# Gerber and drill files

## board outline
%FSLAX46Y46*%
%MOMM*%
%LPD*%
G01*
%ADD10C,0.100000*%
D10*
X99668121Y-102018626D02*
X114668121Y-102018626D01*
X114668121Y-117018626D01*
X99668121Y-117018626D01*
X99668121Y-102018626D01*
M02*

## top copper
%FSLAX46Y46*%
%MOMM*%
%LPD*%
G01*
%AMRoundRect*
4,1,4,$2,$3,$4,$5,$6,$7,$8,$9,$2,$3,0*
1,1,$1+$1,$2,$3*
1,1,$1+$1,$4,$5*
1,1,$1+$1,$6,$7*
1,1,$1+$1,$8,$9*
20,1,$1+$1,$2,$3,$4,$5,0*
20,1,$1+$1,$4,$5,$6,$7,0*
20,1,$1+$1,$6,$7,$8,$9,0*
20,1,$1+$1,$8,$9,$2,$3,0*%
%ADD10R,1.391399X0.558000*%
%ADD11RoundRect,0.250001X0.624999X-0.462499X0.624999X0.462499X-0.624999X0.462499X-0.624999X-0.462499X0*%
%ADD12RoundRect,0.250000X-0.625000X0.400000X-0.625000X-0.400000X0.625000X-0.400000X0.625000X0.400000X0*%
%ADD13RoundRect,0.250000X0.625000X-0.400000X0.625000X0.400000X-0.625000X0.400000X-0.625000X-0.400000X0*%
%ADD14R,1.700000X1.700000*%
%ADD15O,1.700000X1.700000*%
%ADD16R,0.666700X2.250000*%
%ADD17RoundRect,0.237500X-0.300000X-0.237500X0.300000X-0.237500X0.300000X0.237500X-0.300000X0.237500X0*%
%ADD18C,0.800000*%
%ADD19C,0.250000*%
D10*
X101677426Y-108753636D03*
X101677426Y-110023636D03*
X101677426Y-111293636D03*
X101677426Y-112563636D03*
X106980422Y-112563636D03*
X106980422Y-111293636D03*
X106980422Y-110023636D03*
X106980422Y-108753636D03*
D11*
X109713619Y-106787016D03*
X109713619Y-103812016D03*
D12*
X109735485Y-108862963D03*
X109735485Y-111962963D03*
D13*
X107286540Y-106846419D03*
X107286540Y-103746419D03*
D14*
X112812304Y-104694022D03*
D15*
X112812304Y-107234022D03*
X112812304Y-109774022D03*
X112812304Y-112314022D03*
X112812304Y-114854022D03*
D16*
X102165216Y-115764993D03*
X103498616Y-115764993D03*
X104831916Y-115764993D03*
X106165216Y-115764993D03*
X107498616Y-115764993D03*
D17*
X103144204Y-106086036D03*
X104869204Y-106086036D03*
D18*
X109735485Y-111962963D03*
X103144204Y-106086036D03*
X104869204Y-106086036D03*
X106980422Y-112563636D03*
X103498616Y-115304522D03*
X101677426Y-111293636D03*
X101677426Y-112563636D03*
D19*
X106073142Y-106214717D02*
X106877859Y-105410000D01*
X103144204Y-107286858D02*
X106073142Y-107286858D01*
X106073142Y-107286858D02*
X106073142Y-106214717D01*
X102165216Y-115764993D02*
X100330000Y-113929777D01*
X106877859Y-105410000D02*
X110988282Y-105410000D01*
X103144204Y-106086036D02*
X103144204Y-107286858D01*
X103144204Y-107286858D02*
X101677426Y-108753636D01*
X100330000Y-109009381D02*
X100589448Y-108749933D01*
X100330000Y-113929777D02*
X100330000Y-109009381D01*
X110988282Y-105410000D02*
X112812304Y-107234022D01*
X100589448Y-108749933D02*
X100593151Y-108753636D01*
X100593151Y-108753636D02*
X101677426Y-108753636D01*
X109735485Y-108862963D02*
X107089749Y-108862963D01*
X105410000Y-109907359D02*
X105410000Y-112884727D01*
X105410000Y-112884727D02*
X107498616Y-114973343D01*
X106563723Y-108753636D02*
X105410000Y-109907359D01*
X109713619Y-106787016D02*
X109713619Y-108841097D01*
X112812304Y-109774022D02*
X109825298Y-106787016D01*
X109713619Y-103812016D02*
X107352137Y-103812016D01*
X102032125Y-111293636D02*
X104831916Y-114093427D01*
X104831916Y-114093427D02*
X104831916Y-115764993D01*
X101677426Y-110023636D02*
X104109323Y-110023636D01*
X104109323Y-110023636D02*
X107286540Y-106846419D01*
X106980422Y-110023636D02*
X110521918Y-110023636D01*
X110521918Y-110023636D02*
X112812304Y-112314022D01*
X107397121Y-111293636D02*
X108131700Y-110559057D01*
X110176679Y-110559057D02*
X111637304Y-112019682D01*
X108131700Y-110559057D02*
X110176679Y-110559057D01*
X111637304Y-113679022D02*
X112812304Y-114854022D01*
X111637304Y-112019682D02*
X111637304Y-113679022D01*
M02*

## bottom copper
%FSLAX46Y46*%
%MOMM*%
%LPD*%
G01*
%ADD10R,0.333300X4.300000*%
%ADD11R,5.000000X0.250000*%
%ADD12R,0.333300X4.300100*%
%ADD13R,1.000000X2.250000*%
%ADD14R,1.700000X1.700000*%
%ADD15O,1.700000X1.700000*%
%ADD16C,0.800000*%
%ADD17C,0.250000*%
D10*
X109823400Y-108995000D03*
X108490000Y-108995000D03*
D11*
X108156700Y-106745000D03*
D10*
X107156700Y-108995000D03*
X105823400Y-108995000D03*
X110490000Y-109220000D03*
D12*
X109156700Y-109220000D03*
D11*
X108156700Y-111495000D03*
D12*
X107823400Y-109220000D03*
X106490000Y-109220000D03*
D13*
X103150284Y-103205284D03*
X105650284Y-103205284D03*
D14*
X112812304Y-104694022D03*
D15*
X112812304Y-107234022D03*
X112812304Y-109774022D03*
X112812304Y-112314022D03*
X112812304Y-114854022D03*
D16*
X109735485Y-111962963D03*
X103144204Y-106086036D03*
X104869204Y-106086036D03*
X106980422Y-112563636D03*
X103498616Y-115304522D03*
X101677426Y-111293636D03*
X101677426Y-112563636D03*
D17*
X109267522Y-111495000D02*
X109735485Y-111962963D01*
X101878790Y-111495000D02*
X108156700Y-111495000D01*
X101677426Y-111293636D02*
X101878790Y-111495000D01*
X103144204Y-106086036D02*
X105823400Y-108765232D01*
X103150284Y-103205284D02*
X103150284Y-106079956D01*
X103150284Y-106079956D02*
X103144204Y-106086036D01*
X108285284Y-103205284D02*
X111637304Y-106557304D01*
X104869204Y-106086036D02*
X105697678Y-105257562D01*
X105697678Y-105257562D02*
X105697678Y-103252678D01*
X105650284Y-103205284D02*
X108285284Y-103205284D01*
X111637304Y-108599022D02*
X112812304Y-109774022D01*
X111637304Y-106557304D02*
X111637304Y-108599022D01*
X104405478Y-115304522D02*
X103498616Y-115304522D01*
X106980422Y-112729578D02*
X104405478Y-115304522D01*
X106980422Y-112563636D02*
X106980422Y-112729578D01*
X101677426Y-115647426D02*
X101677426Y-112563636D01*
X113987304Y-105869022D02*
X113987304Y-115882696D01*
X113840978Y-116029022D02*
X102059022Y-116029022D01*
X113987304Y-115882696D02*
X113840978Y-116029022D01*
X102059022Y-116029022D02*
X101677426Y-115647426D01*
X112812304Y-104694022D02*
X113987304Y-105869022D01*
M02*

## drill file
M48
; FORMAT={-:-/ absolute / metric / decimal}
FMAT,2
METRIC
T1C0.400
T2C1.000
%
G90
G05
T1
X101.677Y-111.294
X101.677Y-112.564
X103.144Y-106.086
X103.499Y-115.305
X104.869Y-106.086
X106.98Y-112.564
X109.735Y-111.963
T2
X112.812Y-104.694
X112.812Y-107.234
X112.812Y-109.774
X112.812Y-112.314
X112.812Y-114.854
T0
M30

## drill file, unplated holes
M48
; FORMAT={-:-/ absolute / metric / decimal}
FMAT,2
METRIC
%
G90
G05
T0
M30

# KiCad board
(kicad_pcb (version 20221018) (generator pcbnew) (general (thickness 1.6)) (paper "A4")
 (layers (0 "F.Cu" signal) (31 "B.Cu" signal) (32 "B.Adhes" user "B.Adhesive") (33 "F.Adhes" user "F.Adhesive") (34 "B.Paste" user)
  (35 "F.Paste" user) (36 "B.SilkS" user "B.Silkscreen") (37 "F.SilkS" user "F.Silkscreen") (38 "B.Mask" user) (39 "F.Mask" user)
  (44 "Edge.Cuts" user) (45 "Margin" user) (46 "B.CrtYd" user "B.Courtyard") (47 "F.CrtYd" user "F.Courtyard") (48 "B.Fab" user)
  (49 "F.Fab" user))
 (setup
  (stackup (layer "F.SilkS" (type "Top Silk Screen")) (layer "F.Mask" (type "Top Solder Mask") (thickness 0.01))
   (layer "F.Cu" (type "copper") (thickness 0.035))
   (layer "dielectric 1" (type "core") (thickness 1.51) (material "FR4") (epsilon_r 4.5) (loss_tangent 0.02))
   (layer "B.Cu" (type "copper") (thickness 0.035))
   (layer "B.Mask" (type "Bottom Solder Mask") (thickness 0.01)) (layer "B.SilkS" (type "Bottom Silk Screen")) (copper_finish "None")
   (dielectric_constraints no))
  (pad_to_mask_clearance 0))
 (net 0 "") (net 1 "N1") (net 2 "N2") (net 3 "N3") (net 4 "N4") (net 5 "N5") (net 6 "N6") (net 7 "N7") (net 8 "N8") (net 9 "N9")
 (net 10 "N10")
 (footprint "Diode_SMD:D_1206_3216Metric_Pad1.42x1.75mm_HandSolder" (layer "F.Cu") (at 109.713619 105.299516 90)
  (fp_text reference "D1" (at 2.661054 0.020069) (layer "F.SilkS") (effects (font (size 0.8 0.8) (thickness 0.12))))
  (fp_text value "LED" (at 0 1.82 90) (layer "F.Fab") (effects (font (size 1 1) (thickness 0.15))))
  (pad "1" smd roundrect (at -1.4875 0 90) (size 1.425 1.75) (layers "F.Cu" "F.Paste" "F.Mask") (roundrect_rratio 0.1754392982) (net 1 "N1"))
  (pad "2" smd roundrect (at 1.4875 0 90) (size 1.425 1.75) (layers "F.Cu" "F.Paste" "F.Mask") (roundrect_rratio 0.1754392982) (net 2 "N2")))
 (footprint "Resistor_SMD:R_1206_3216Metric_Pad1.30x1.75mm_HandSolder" (layer "F.Cu") (at 109.735485 110.412963 -90)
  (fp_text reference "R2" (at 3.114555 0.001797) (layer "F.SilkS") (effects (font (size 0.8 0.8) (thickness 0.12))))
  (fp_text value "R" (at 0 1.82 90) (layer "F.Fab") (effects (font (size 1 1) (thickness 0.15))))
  (pad "1" smd roundrect (at -1.55 0 270) (size 1.3 1.75) (layers "F.Cu" "F.Paste" "F.Mask") (roundrect_rratio 0.1923076923) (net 1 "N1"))
  (pad "2" smd roundrect (at 1.55 0 270) (size 1.3 1.75) (layers "F.Cu" "F.Paste" "F.Mask") (roundrect_rratio 0.1923076923) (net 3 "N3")))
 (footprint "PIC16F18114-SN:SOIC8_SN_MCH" (layer "F.Cu") (at 104.328924 110.658636)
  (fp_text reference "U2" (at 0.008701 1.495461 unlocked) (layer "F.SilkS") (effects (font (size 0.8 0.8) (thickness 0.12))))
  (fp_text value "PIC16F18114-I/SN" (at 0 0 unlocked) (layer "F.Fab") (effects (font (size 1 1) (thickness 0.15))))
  (pad "1" smd rect (at -2.651498 -1.905) (size 1.391399 0.558) (layers "F.Cu" "F.Paste" "F.Mask") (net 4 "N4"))
  (pad "2" smd rect (at -2.651498 -0.635) (size 1.391399 0.558) (layers "F.Cu" "F.Paste" "F.Mask") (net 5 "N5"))
  (pad "3" smd rect (at -2.651498 0.635) (size 1.391399 0.558) (layers "F.Cu" "F.Paste" "F.Mask") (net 3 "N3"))
  (pad "4" smd rect (at -2.651498 1.905) (size 1.391399 0.558) (layers "F.Cu" "F.Paste" "F.Mask") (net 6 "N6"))
  (pad "5" smd rect (at 2.651498 1.905) (size 1.391399 0.558) (layers "F.Cu" "F.Paste" "F.Mask") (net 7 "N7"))
  (pad "6" smd rect (at 2.651498 0.635) (size 1.391399 0.558) (layers "F.Cu" "F.Paste" "F.Mask") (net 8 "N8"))
  (pad "7" smd rect (at 2.651498 -0.635) (size 1.391399 0.558) (layers "F.Cu" "F.Paste" "F.Mask") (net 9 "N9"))
  (pad "8" smd rect (at 2.651498 -1.905) (size 1.391399 0.558) (layers "F.Cu" "F.Paste" "F.Mask") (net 1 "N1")))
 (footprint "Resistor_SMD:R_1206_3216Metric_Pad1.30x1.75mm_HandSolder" (layer "F.Cu") (at 107.28654 105.296419 90)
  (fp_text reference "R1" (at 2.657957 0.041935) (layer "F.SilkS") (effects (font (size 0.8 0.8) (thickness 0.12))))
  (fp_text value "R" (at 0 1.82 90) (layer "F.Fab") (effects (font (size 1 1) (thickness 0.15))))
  (pad "1" smd roundrect (at -1.55 0 90) (size 1.3 1.75) (layers "F.Cu" "F.Paste" "F.Mask") (roundrect_rratio 0.1923076923) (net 5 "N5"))
  (pad "2" smd roundrect (at 1.55 0 90) (size 1.3 1.75) (layers "F.Cu" "F.Paste" "F.Mask") (roundrect_rratio 0.1923076923) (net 2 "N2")))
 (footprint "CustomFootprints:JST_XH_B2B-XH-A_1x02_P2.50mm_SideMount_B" (layer "F.Cu") (at 103.150284 103.205284)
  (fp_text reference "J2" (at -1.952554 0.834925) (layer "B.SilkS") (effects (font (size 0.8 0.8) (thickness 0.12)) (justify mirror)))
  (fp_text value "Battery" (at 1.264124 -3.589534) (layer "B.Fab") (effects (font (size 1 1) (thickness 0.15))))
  (pad "1" smd rect (at 0 0) (size 1 2.25) (layers "B.Cu" "B.Paste" "B.Mask") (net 4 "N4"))
  (pad "2" smd rect (at 2.5 0) (size 1 2.25) (layers "B.Cu" "B.Paste" "B.Mask") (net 1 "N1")))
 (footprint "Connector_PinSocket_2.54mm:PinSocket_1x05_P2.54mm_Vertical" (layer "F.Cu") (at 112.812304 104.694022)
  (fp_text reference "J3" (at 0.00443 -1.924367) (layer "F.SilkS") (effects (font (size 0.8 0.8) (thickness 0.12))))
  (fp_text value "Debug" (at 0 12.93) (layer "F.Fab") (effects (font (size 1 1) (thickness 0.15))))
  (pad "1" thru_hole rect (at 0 0) (size 1.7 1.7) (drill 1) (layers "*.Cu" "*.Mask") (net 6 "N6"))
  (pad "2" thru_hole oval (at 0 2.54) (size 1.7 1.7) (drill 1) (layers "*.Cu" "*.Mask") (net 4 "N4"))
  (pad "3" thru_hole oval (at 0 5.08) (size 1.7 1.7) (drill 1) (layers "*.Cu" "*.Mask") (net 1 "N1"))
  (pad "4" thru_hole oval (at 0 7.62) (size 1.7 1.7) (drill 1) (layers "*.Cu" "*.Mask") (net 9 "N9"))
  (pad "5" thru_hole oval (at 0 10.16) (size 1.7 1.7) (drill 1) (layers "*.Cu" "*.Mask") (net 8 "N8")))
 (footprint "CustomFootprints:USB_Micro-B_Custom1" (layer "F.Cu") (at 104.831916 116.364993)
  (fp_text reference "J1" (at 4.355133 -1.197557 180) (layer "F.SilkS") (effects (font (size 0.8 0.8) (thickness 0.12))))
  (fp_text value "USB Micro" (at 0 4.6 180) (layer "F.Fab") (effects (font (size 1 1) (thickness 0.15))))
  (pad "1" smd rect (at -2.6667 -0.6) (size 0.6667 2.25) (layers "F.Cu" "F.Paste" "F.Mask") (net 4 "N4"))
  (pad "2" smd rect (at -1.3333 -0.6) (size 0.6667 2.25) (layers "F.Cu" "F.Paste" "F.Mask") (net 7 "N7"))
  (pad "3" smd rect (at 0 -0.6) (size 0.6667 2.25) (layers "F.Cu" "F.Paste" "F.Mask") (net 3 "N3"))
  (pad "4" smd rect (at 1.3333 -0.6) (size 0.6667 2.25) (layers "F.Cu" "F.Paste" "F.Mask") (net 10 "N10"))
  (pad "5" smd rect (at 2.6667 -0.6) (size 0.6667 2.25) (layers "F.Cu" "F.Paste" "F.Mask") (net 1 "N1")))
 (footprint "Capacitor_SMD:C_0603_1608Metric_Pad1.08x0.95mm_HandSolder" (layer "F.Cu") (at 104.006704 106.086036)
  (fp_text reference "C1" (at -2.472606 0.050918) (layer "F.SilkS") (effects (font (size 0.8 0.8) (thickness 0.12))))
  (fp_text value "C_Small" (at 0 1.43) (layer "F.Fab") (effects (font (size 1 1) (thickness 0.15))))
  (pad "1" smd roundrect (at -0.8625 0) (size 1.075 0.95) (layers "F.Cu" "F.Paste" "F.Mask") (roundrect_rratio 0.25) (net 4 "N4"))
  (pad "2" smd roundrect (at 0.8625 0) (size 1.075 0.95) (layers "F.Cu" "F.Paste" "F.Mask") (roundrect_rratio 0.25) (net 1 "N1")))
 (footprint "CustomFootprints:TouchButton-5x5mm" (layer "B.Cu") (at 108.1567 109.12 180)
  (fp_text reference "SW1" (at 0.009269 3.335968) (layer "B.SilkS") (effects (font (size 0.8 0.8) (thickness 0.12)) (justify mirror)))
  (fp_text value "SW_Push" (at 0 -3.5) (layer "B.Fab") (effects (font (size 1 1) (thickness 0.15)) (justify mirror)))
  (pad "1" smd rect (at -1.6667 0.125 180) (size 0.3333 4.3) (layers "B.Cu" "B.Paste" "B.Mask") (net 4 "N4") (thermal_bridge_angle 45))
  (pad "1" smd rect (at -0.3333 0.125 180) (size 0.3333 4.3) (layers "B.Cu" "B.Paste" "B.Mask") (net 4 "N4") (thermal_bridge_angle 45))
  (pad "1" smd rect (at 0 2.375 180) (size 5 0.25) (layers "B.Cu" "B.Paste" "B.Mask") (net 4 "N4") (thermal_bridge_angle 45))
  (pad "1" smd rect (at 1 0.125 180) (size 0.3333 4.3) (layers "B.Cu" "B.Paste" "B.Mask") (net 4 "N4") (thermal_bridge_angle 45))
  (pad "1" smd rect (at 2.3333 0.125 180) (size 0.3333 4.3) (layers "B.Cu" "B.Paste" "B.Mask") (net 4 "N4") (thermal_bridge_angle 45))
  (pad "2" smd rect (at -2.3333 -0.1 180) (size 0.3333 4.3) (layers "B.Cu" "B.Paste" "B.Mask") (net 3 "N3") (thermal_bridge_angle 45))
  (pad "2" smd rect (at -1 -0.1 180) (size 0.3333 4.3001) (layers "B.Cu" "B.Paste" "B.Mask") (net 3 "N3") (thermal_bridge_angle 45))
  (pad "2" smd rect (at 0 -2.375 180) (size 5 0.25) (layers "B.Cu" "B.Paste" "B.Mask") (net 3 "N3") (thermal_bridge_angle 45))
  (pad "2" smd rect (at 0.3333 -0.1 180) (size 0.3333 4.3001) (layers "B.Cu" "B.Paste" "B.Mask") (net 3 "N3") (thermal_bridge_angle 45))
  (pad "2" smd rect (at 1.6667 -0.1 180) (size 0.3333 4.3001) (layers "B.Cu" "B.Paste" "B.Mask") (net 3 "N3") (thermal_bridge_angle 45)))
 (gr_rect (start 99.668121 102.018626) (end 114.668121 117.018626) (stroke (width 0.1) (type default)) (fill none) (layer "Edge.Cuts"))
 (segment (start 102.165216 115.764993) (end 100.33 113.929777) (width 0.25) (layer "F.Cu") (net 4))
 (segment (start 106.877859 105.41) (end 110.988282 105.41) (width 0.25) (layer "F.Cu") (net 4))
 (segment (start 103.144204 106.086036) (end 103.144204 107.286858) (width 0.25) (layer "F.Cu") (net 4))
 (segment (start 103.144204 107.286858) (end 106.073142 107.286858) (width 0.25) (layer "F.Cu") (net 4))
 (segment (start 106.073142 106.214717) (end 106.877859 105.41) (width 0.25) (layer "F.Cu") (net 4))
 (segment (start 103.144204 107.286858) (end 101.677426 108.753636) (width 0.25) (layer "F.Cu") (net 4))
 (segment (start 100.33 109.009381) (end 100.589448 108.749933) (width 0.25) (layer "F.Cu") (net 4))
 (segment (start 100.33 113.929777) (end 100.33 109.009381) (width 0.25) (layer "F.Cu") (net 4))
 (segment (start 110.988282 105.41) (end 112.812304 107.234022) (width 0.25) (layer "F.Cu") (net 4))
 (segment (start 106.073142 107.286858) (end 106.073142 106.214717) (width 0.25) (layer "F.Cu") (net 4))
 (segment (start 100.589448 108.749933) (end 100.593151 108.753636) (width 0.25) (layer "F.Cu") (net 4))
 (segment (start 100.593151 108.753636) (end 101.677426 108.753636) (width 0.25) (layer "F.Cu") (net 4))
 (via (at 103.144204 106.086036) (size 0.8) (drill 0.4) (layers "F.Cu" "B.Cu") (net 4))
 (segment (start 103.150284 103.205284) (end 103.150284 106.079956) (width 0.25) (layer "B.Cu") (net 4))
 (segment (start 103.150284 106.079956) (end 103.144204 106.086036) (width 0.25) (layer "B.Cu") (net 4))
 (segment (start 103.144204 106.086036) (end 105.8234 108.765232) (width 0.25) (layer "B.Cu") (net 4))
 (segment (start 109.735485 108.862963) (end 107.089749 108.862963) (width 0.25) (layer "F.Cu") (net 1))
 (segment (start 105.41 109.907359) (end 105.41 112.884727) (width 0.25) (layer "F.Cu") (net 1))
 (segment (start 105.41 112.884727) (end 107.498616 114.973343) (width 0.25) (layer "F.Cu") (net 1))
 (segment (start 106.563723 108.753636) (end 105.41 109.907359) (width 0.25) (layer "F.Cu") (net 1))
 (segment (start 109.713619 106.787016) (end 109.713619 108.841097) (width 0.25) (layer "F.Cu") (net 1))
 (segment (start 112.812304 109.774022) (end 109.825298 106.787016) (width 0.25) (layer "F.Cu") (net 1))
 (via (at 104.869204 106.086036) (size 0.8) (drill 0.4) (layers "F.Cu" "B.Cu") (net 1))
 (segment (start 108.285284 103.205284) (end 111.637304 106.557304) (width 0.25) (layer "B.Cu") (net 1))
 (segment (start 104.869204 106.086036) (end 105.697678 105.257562) (width 0.25) (layer "B.Cu") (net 1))
 (segment (start 105.697678 105.257562) (end 105.697678 103.252678) (width 0.25) (layer "B.Cu") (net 1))
 (segment (start 105.650284 103.205284) (end 108.285284 103.205284) (width 0.25) (layer "B.Cu") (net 1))
 (segment (start 111.637304 108.599022) (end 112.812304 109.774022) (width 0.25) (layer "B.Cu") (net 1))
 (segment (start 111.637304 106.557304) (end 111.637304 108.599022) (width 0.25) (layer "B.Cu") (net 1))
 (segment (start 109.713619 103.812016) (end 107.352137 103.812016) (width 0.25) (layer "F.Cu") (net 2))
 (via (at 106.980422 112.563636) (size 0.8) (drill 0.4) (layers "F.Cu" "B.Cu") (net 7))
 (via (at 103.498616 115.304522) (size 0.8) (drill 0.4) (layers "F.Cu" "B.Cu") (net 7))
 (segment (start 104.405478 115.304522) (end 103.498616 115.304522) (width 0.25) (layer "B.Cu") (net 7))
 (segment (start 106.980422 112.729578) (end 104.405478 115.304522) (width 0.25) (layer "B.Cu") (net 7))
 (segment (start 106.980422 112.563636) (end 106.980422 112.729578) (width 0.25) (layer "B.Cu") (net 7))
 (segment (start 102.032125 111.293636) (end 104.831916 114.093427) (width 0.25) (layer "F.Cu") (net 3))
 (segment (start 104.831916 114.093427) (end 104.831916 115.764993) (width 0.25) (layer "F.Cu") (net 3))
 (via (at 101.677426 111.293636) (size 0.8) (drill 0.4) (layers "F.Cu" "B.Cu") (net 3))
 (via (at 109.735485 111.962963) (size 0.8) (drill 0.4) (layers "F.Cu" "B.Cu") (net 3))
 (segment (start 109.267522 111.495) (end 109.735485 111.962963) (width 0.25) (layer "B.Cu") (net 3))
 (segment (start 101.87879 111.495) (end 108.1567 111.495) (width 0.25) (layer "B.Cu") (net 3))
 (segment (start 101.677426 111.293636) (end 101.87879 111.495) (width 0.25) (layer "B.Cu") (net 3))
 (segment (start 101.677426 110.023636) (end 104.109323 110.023636) (width 0.25) (layer "F.Cu") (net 5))
 (segment (start 104.109323 110.023636) (end 107.28654 106.846419) (width 0.25) (layer "F.Cu") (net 5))
 (via (at 101.677426 112.563636) (size 0.8) (drill 0.4) (layers "F.Cu" "B.Cu") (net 6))
 (segment (start 101.677426 115.647426) (end 101.677426 112.563636) (width 0.25) (layer "B.Cu") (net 6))
 (segment (start 113.987304 105.869022) (end 113.987304 115.882696) (width 0.25) (layer "B.Cu") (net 6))
 (segment (start 113.840978 116.029022) (end 102.059022 116.029022) (width 0.25) (layer "B.Cu") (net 6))
 (segment (start 113.987304 115.882696) (end 113.840978 116.029022) (width 0.25) (layer "B.Cu") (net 6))
 (segment (start 102.059022 116.029022) (end 101.677426 115.647426) (width 0.25) (layer "B.Cu") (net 6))
 (segment (start 112.812304 104.694022) (end 113.987304 105.869022) (width 0.25) (layer "B.Cu") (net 6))
 (segment (start 106.980422 110.023636) (end 110.521918 110.023636) (width 0.25) (layer "F.Cu") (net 9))
 (segment (start 110.521918 110.023636) (end 112.812304 112.314022) (width 0.25) (layer "F.Cu") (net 9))
 (segment (start 107.397121 111.293636) (end 108.1317 110.559057) (width 0.25) (layer "F.Cu") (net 8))
 (segment (start 110.176679 110.559057) (end 111.637304 112.019682) (width 0.25) (layer "F.Cu") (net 8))
 (segment (start 108.1317 110.559057) (end 110.176679 110.559057) (width 0.25) (layer "F.Cu") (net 8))
 (segment (start 111.637304 113.679022) (end 112.812304 114.854022) (width 0.25) (layer "F.Cu") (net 8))
 (segment (start 111.637304 112.019682) (end 111.637304 113.679022) (width 0.25) (layer "F.Cu") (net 8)))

